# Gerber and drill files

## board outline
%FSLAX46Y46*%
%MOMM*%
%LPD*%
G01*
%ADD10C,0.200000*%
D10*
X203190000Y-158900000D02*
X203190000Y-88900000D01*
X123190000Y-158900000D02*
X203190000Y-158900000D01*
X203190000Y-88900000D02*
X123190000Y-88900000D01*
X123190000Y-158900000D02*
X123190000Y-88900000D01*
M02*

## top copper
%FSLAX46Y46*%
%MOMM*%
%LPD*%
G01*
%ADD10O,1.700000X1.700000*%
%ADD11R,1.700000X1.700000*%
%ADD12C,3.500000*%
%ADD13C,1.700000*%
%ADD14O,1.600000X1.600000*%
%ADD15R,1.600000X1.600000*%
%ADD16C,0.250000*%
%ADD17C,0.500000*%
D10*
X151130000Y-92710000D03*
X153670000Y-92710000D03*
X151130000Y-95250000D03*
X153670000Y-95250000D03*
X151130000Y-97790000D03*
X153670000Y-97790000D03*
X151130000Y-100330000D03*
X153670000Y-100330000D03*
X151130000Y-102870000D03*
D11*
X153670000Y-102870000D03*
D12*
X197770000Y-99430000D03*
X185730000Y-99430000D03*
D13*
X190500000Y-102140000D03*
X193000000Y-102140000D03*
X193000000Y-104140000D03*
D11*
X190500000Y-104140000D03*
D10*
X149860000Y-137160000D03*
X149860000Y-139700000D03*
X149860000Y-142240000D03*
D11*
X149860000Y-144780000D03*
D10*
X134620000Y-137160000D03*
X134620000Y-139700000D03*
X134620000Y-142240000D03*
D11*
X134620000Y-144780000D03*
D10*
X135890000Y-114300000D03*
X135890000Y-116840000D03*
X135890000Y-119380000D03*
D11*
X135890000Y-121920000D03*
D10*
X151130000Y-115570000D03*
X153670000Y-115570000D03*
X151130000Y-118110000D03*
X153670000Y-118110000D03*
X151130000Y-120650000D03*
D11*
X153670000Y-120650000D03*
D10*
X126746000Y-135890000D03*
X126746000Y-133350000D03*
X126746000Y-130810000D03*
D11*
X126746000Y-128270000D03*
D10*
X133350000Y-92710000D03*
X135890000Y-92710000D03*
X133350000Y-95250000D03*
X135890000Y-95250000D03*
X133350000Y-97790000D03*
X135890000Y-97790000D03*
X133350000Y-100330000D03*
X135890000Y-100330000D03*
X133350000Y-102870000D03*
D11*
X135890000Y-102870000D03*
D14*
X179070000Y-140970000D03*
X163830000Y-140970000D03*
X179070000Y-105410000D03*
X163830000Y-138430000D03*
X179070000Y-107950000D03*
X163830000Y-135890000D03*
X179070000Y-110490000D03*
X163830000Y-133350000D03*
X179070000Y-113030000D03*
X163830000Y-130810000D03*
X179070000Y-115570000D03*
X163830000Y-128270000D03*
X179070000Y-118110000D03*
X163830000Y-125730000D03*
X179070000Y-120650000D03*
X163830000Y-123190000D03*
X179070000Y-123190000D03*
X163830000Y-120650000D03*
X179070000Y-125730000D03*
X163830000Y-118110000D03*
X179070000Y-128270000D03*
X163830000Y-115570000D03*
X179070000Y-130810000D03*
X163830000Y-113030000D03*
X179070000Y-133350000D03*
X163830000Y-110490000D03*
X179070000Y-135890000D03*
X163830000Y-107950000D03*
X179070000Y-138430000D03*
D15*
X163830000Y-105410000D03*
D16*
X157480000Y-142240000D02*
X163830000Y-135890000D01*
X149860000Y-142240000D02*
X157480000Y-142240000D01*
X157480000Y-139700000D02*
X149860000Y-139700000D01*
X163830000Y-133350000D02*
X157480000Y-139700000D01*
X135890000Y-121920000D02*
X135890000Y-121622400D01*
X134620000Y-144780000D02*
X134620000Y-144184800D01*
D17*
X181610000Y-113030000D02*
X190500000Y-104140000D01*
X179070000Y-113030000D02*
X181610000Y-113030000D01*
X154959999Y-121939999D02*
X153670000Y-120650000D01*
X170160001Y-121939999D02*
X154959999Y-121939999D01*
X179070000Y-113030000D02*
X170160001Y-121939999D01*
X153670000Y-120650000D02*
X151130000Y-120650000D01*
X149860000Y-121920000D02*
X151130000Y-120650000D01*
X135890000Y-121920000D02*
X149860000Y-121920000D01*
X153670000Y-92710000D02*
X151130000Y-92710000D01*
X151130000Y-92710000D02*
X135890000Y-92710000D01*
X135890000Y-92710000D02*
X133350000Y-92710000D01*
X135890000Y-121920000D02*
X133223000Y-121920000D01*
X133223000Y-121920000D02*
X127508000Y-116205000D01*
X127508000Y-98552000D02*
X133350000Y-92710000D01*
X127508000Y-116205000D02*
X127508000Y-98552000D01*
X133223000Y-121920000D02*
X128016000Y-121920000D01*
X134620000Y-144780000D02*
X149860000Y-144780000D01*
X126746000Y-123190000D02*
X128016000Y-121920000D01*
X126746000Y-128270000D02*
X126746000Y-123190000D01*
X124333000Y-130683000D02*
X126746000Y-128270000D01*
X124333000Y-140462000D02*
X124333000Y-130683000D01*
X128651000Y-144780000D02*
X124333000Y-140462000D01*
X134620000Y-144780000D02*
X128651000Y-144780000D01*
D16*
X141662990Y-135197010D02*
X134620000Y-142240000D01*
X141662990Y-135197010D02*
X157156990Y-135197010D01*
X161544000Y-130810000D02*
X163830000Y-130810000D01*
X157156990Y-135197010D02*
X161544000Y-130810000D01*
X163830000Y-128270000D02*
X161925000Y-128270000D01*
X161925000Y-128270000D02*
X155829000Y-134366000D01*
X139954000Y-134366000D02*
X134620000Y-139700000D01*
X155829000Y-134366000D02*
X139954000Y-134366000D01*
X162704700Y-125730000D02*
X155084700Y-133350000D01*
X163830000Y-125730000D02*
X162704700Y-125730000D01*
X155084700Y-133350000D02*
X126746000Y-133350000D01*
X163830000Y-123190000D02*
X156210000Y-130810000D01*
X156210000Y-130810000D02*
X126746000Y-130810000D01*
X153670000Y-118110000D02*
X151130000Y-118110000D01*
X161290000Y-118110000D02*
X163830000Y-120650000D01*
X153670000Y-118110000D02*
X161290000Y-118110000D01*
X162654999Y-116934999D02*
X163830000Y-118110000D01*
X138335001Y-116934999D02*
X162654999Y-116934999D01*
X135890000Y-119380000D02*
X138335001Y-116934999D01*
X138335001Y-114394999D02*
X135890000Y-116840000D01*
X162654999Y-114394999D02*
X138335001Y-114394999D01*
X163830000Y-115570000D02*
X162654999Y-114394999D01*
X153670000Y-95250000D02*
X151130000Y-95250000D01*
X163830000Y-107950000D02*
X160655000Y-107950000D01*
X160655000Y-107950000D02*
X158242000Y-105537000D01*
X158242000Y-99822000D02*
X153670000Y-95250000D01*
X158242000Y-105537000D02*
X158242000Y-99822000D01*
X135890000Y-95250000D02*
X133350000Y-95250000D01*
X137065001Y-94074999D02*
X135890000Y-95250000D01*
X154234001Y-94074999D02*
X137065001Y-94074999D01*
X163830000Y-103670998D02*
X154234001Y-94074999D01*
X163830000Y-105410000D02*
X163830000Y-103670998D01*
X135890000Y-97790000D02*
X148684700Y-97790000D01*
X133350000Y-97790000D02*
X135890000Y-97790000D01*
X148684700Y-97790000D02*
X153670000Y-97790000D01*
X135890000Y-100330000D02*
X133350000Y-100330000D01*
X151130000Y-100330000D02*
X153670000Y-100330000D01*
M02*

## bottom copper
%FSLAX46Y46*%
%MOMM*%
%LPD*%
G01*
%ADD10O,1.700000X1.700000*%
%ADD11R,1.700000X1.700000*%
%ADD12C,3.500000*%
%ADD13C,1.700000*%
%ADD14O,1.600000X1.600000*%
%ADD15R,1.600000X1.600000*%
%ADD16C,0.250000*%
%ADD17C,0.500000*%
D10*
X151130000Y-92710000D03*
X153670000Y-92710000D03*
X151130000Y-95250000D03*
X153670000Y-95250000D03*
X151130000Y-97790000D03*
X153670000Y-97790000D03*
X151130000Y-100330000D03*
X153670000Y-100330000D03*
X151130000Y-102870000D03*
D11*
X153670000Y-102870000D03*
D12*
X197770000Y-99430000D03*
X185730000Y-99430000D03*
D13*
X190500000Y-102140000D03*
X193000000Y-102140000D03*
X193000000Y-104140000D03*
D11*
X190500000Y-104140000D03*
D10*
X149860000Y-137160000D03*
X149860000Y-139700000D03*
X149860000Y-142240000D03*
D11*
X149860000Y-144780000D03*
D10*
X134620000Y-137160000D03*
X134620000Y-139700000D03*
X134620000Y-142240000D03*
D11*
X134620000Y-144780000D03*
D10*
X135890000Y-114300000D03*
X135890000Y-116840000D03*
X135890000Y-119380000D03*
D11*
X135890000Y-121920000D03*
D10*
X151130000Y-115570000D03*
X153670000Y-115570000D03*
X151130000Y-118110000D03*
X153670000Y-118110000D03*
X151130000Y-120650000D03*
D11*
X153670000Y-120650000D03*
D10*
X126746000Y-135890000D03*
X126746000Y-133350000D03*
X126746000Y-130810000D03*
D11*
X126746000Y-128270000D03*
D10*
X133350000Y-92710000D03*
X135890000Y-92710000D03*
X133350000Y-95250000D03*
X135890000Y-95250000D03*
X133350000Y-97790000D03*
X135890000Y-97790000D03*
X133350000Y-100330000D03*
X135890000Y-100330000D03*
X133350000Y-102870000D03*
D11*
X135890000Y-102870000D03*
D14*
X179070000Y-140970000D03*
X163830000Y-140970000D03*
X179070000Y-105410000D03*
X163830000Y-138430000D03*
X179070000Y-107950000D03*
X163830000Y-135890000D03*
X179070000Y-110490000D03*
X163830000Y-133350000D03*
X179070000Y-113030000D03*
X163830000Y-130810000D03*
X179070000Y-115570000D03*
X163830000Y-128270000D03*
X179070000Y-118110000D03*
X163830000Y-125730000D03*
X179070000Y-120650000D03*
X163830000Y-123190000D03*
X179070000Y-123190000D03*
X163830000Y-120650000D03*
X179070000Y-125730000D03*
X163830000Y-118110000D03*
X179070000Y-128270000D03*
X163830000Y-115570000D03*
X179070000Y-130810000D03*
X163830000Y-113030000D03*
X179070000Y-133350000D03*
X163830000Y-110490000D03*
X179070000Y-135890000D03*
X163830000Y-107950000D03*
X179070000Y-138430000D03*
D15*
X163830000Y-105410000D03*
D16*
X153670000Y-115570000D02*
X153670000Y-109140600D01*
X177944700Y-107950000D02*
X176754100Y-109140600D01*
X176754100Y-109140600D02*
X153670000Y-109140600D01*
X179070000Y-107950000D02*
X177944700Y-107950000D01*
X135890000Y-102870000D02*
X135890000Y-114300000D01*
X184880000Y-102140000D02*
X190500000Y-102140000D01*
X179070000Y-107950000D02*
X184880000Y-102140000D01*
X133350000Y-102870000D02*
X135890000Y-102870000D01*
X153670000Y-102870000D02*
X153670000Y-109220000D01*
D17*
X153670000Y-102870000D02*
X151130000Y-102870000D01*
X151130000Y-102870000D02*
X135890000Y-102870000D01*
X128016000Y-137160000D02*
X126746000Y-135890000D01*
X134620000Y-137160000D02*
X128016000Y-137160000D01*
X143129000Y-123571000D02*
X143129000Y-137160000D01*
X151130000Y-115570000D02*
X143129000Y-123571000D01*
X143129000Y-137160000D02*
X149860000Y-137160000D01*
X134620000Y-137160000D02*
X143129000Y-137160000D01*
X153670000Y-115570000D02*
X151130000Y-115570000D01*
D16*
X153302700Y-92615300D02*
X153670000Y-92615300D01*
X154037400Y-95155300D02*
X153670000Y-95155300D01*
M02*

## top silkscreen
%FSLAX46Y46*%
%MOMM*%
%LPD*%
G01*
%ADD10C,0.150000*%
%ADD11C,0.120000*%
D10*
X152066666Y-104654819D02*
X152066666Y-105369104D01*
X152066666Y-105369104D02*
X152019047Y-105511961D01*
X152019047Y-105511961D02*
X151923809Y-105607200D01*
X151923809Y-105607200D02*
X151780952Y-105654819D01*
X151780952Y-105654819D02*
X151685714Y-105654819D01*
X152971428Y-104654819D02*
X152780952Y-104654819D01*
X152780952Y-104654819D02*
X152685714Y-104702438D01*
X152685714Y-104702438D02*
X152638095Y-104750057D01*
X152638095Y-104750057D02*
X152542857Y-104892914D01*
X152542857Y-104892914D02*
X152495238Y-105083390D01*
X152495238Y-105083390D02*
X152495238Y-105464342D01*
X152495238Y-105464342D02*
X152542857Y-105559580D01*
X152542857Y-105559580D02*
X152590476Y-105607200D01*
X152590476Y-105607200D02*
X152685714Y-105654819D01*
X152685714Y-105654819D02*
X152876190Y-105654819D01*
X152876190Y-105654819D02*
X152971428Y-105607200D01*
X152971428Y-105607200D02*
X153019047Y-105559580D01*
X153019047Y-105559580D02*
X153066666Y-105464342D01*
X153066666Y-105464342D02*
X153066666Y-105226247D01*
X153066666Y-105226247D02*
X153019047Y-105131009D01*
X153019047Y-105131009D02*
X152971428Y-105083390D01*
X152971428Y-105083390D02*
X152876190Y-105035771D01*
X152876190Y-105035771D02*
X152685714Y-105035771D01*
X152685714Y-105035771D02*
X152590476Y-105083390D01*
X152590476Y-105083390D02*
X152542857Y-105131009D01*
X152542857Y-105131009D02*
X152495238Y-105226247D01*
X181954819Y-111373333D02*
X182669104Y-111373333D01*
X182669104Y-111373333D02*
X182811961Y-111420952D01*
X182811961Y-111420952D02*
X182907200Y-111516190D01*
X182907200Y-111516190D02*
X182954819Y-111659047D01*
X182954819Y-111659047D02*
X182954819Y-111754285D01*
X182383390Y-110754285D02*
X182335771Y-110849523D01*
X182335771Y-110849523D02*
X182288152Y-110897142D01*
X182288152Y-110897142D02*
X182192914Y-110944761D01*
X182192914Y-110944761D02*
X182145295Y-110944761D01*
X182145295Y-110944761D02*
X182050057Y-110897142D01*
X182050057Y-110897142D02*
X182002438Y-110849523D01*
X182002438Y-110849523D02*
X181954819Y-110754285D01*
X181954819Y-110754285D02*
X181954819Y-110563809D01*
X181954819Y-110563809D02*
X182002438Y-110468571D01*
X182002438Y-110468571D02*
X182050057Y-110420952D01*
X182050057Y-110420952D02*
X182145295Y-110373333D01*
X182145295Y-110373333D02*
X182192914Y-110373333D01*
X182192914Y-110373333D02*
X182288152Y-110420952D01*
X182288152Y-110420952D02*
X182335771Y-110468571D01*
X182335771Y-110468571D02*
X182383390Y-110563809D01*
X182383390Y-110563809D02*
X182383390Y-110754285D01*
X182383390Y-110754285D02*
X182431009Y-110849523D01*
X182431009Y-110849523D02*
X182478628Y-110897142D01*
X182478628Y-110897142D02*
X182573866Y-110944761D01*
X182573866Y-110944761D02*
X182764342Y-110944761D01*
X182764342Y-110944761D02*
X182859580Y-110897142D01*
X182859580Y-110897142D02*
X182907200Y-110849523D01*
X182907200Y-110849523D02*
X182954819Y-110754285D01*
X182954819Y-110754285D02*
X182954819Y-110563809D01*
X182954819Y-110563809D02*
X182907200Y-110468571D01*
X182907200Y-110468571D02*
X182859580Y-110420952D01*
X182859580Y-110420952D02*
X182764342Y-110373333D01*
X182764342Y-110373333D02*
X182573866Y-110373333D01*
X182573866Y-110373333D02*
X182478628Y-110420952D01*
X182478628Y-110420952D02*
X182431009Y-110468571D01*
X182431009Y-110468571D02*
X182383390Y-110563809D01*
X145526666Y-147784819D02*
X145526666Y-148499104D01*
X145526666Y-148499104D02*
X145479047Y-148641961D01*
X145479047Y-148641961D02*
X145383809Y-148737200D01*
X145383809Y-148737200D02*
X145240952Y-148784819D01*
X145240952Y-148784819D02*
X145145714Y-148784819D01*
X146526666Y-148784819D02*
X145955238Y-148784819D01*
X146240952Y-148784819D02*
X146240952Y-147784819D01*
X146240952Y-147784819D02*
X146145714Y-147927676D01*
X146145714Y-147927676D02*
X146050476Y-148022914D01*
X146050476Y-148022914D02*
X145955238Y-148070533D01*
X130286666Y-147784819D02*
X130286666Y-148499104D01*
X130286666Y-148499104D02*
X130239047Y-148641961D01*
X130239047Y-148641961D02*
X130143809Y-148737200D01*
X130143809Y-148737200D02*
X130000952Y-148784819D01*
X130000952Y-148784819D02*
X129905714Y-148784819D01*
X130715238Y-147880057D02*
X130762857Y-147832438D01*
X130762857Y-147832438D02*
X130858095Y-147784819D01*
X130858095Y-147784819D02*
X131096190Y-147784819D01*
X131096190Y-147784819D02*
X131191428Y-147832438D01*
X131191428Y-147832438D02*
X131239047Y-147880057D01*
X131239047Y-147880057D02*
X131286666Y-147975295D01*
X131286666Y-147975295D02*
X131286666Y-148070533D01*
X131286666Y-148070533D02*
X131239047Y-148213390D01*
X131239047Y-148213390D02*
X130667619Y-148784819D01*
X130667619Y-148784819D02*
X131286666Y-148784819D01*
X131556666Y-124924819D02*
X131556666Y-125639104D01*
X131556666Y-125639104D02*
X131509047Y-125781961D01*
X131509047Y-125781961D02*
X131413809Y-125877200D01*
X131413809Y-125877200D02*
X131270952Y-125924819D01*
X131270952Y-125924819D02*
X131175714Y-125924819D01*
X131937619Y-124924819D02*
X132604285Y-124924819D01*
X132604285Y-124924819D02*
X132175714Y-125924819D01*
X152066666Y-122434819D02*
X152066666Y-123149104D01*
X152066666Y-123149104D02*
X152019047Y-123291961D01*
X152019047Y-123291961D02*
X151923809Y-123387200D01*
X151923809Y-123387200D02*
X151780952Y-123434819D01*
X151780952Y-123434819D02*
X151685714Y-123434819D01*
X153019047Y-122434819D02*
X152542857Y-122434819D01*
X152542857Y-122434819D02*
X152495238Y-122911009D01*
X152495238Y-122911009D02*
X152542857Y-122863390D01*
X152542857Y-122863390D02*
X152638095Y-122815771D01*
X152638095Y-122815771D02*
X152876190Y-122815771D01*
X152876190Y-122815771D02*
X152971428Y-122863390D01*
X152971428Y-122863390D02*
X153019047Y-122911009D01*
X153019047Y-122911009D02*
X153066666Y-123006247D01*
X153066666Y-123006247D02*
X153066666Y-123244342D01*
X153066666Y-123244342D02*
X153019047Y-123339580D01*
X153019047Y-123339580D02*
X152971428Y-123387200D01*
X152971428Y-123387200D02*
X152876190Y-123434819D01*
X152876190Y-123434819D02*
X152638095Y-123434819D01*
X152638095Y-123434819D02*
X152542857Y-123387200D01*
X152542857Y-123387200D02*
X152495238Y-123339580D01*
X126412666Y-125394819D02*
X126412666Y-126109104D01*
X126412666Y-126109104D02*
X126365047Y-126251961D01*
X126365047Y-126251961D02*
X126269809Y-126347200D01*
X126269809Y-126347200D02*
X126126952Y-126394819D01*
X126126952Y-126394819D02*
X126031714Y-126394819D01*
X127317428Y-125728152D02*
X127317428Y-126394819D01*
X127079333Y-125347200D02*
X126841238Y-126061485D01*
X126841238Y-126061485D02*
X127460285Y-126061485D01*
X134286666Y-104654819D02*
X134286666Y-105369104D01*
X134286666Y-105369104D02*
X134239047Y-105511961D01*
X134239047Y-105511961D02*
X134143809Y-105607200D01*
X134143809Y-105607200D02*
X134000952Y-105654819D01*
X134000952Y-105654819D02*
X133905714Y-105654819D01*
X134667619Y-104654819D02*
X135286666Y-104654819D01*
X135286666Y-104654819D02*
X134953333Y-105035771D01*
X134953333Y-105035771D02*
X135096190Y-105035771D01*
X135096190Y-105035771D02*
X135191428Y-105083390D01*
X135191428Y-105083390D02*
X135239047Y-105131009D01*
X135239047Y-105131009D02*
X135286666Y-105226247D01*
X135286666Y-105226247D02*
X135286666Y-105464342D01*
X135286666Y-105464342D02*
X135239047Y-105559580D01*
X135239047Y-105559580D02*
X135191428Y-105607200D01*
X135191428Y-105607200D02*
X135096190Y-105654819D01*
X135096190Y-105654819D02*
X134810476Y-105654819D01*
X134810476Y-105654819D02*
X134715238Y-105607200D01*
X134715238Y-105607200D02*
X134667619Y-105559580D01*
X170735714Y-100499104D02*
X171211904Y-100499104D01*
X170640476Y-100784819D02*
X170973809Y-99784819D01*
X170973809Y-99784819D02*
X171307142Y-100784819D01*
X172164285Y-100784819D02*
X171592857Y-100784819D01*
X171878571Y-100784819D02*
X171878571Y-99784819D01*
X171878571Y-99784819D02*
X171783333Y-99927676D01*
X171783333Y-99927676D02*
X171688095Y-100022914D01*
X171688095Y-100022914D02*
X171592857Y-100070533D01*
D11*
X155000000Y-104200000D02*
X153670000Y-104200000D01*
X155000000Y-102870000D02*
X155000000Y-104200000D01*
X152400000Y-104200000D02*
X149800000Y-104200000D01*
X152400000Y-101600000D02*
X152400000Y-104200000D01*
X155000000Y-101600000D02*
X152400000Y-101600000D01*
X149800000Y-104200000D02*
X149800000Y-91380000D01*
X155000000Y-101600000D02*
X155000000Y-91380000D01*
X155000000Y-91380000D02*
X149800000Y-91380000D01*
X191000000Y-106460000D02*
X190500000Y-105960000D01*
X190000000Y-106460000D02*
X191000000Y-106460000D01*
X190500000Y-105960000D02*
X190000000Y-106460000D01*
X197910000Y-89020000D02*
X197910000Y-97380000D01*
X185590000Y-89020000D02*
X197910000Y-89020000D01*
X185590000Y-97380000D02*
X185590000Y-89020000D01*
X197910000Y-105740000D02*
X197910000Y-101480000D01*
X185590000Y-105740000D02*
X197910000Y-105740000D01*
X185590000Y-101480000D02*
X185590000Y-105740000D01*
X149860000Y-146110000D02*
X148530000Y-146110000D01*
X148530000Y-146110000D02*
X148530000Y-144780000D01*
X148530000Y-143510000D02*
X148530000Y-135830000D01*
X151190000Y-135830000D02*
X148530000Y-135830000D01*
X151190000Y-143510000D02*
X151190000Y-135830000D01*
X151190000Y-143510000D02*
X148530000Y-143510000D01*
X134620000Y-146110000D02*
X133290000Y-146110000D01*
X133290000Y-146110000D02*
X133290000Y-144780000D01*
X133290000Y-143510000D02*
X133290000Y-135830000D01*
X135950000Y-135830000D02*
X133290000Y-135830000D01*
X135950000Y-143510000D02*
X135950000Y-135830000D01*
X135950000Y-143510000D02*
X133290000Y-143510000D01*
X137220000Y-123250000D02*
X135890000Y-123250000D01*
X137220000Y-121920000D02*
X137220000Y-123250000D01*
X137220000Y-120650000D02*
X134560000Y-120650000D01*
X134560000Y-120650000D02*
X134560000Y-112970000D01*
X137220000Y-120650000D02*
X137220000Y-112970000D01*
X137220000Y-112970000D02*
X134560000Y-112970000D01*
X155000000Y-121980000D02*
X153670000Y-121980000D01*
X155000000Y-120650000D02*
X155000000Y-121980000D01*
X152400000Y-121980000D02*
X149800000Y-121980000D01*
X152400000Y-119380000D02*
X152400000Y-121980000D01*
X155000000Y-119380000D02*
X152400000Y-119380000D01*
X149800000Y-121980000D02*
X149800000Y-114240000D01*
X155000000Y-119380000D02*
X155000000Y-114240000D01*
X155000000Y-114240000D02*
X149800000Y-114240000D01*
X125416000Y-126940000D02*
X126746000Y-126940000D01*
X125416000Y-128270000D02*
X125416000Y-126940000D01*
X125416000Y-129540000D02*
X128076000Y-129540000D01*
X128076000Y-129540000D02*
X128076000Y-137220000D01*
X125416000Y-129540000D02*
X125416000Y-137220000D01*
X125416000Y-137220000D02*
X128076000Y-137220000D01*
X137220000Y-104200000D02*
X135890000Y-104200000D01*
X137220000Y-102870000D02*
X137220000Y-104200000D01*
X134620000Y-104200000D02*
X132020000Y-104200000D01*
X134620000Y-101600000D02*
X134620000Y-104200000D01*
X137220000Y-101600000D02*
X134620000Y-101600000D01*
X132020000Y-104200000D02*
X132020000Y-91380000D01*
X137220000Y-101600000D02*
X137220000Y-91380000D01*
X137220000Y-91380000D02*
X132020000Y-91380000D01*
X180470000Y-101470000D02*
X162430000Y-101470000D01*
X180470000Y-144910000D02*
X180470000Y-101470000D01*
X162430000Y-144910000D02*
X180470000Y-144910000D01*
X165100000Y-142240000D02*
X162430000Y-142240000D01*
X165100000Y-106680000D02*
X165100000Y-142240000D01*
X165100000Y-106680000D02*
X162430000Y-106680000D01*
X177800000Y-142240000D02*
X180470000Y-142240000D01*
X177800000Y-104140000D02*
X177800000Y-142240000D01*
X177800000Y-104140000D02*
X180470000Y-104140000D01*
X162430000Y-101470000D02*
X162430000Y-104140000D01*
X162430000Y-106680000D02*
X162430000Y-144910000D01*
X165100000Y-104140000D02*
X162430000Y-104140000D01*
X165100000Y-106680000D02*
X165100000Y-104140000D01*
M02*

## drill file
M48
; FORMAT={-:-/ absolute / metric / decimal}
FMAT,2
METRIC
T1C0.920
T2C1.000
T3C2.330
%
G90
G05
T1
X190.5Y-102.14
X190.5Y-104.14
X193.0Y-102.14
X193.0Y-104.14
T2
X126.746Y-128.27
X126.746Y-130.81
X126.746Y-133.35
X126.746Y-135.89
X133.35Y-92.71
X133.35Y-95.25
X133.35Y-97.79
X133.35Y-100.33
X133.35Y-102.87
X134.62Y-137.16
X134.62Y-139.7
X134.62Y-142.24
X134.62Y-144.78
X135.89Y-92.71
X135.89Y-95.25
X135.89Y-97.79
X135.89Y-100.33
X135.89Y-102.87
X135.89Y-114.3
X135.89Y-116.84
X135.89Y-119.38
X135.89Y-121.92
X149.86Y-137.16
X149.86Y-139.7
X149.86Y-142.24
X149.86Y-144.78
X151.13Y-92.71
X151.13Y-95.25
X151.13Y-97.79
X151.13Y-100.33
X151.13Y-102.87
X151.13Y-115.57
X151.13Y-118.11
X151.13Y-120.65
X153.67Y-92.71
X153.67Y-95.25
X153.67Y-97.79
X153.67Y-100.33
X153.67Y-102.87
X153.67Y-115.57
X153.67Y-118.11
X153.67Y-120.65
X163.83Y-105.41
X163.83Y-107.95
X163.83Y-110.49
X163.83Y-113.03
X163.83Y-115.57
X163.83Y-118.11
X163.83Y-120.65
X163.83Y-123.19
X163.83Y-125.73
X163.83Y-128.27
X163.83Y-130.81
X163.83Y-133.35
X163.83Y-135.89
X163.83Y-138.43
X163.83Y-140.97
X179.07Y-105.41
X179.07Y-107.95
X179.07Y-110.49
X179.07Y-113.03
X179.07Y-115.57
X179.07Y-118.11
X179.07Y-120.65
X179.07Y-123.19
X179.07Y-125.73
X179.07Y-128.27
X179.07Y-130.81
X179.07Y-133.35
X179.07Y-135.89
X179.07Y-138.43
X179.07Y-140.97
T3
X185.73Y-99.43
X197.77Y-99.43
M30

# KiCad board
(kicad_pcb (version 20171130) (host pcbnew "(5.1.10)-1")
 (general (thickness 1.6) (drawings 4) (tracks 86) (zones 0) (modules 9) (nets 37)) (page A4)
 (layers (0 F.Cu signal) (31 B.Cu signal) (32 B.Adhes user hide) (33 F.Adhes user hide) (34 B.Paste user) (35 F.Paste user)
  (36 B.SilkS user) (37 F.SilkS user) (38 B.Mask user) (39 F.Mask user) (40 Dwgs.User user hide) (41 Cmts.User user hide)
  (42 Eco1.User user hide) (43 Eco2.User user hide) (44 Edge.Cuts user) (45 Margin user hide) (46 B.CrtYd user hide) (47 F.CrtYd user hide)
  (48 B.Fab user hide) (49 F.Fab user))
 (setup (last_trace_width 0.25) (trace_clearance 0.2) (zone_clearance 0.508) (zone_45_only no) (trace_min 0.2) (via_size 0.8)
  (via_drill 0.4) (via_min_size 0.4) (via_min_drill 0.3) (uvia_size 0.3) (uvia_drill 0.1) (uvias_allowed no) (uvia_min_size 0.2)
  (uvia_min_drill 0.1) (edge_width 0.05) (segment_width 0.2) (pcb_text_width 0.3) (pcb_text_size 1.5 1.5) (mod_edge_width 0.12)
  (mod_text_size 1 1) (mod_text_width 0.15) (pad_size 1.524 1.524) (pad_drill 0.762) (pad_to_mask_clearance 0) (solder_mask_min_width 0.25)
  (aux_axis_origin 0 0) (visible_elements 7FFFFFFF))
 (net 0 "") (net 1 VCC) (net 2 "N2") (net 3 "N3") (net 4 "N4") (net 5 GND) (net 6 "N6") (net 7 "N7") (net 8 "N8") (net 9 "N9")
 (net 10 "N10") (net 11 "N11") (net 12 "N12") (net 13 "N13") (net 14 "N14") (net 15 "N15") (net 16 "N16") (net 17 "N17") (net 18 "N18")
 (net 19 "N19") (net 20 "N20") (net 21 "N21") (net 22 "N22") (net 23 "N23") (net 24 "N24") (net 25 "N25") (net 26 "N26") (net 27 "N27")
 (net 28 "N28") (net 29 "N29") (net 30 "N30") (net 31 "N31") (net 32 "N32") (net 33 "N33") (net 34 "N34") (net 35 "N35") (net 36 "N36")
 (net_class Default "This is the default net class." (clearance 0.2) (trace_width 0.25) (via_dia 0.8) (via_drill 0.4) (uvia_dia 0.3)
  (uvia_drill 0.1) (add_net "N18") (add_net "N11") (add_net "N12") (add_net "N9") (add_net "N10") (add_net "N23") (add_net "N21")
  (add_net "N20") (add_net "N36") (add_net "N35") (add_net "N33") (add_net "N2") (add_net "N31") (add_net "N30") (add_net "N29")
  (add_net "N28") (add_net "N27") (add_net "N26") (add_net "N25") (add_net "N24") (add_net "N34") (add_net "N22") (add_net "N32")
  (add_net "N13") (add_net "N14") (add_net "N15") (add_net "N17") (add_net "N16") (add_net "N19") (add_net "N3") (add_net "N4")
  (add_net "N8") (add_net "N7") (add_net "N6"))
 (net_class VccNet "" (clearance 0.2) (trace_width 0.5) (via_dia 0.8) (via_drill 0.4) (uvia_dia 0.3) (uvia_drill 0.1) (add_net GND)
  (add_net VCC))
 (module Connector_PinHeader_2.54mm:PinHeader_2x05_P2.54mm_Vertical (layer F.Cu) (at 153.67 102.87 180)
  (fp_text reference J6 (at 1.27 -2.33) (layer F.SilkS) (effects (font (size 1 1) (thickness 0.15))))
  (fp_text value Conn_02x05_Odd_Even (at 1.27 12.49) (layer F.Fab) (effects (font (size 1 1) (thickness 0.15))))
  (fp_line (start -1.33 -1.33) (end 0 -1.33) (layer F.SilkS) (width 0.12))
  (fp_line (start -1.33 0) (end -1.33 -1.33) (layer F.SilkS) (width 0.12))
  (fp_line (start 1.27 -1.33) (end 3.87 -1.33) (layer F.SilkS) (width 0.12))
  (fp_line (start 1.27 1.27) (end 1.27 -1.33) (layer F.SilkS) (width 0.12))
  (fp_line (start -1.33 1.27) (end 1.27 1.27) (layer F.SilkS) (width 0.12))
  (fp_line (start 3.87 -1.33) (end 3.87 11.49) (layer F.SilkS) (width 0.12))
  (fp_line (start -1.33 1.27) (end -1.33 11.49) (layer F.SilkS) (width 0.12))
  (fp_line (start -1.33 11.49) (end 3.87 11.49) (layer F.SilkS) (width 0.12))
  (pad 10 thru_hole oval (at 2.54 10.16 180) (size 1.7 1.7) (drill 1) (layers *.Cu *.Mask) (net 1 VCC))
  (pad 9 thru_hole oval (at 0 10.16 180) (size 1.7 1.7) (drill 1) (layers *.Cu *.Mask) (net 1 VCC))
  (pad 8 thru_hole oval (at 2.54 7.62 180) (size 1.7 1.7) (drill 1) (layers *.Cu *.Mask) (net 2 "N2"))
  (pad 7 thru_hole oval (at 0 7.62 180) (size 1.7 1.7) (drill 1) (layers *.Cu *.Mask) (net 2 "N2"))
  (pad 6 thru_hole oval (at 2.54 5.08 180) (size 1.7 1.7) (drill 1) (layers *.Cu *.Mask) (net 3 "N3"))
  (pad 5 thru_hole oval (at 0 5.08 180) (size 1.7 1.7) (drill 1) (layers *.Cu *.Mask) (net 3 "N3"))
  (pad 4 thru_hole oval (at 2.54 2.54 180) (size 1.7 1.7) (drill 1) (layers *.Cu *.Mask) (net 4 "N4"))
  (pad 3 thru_hole oval (at 0 2.54 180) (size 1.7 1.7) (drill 1) (layers *.Cu *.Mask) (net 4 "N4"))
  (pad 2 thru_hole oval (at 2.54 0 180) (size 1.7 1.7) (drill 1) (layers *.Cu *.Mask) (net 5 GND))
  (pad 1 thru_hole rect (at 0 0 180) (size 1.7 1.7) (drill 1) (layers *.Cu *.Mask) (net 5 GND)))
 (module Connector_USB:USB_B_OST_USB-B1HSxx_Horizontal (layer F.Cu) (at 190.5 104.14 90)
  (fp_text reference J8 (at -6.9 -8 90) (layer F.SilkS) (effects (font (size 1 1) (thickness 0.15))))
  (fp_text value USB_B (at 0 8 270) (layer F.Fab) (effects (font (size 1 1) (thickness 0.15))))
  (fp_line (start -2.32 0.5) (end -1.82 0) (layer F.SilkS) (width 0.12))
  (fp_line (start -2.32 -0.5) (end -2.32 0.5) (layer F.SilkS) (width 0.12))
  (fp_line (start -1.82 0) (end -2.32 -0.5) (layer F.SilkS) (width 0.12))
  (fp_line (start 15.12 7.41) (end 6.76 7.41) (layer F.SilkS) (width 0.12))
  (fp_line (start 15.12 -4.91) (end 15.12 7.41) (layer F.SilkS) (width 0.12))
  (fp_line (start 6.76 -4.91) (end 15.12 -4.91) (layer F.SilkS) (width 0.12))
  (fp_line (start -1.6 7.41) (end 2.66 7.41) (layer F.SilkS) (width 0.12))
  (fp_line (start -1.6 -4.91) (end -1.6 7.41) (layer F.SilkS) (width 0.12))
  (fp_line (start 2.66 -4.91) (end -1.6 -4.91) (layer F.SilkS) (width 0.12))
  (pad 5 thru_hole circle (at 4.71 7.27 90) (size 3.5 3.5) (drill 2.33) (layers *.Cu *.Mask) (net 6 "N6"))
  (pad 5 thru_hole circle (at 4.71 -4.77 90) (size 3.5 3.5) (drill 2.33) (layers *.Cu *.Mask) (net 6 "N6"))
  (pad 4 thru_hole circle (at 2 0 90) (size 1.7 1.7) (drill 0.92) (layers *.Cu *.Mask) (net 5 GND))
  (pad 3 thru_hole circle (at 2 2.5 90) (size 1.7 1.7) (drill 0.92) (layers *.Cu *.Mask) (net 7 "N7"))
  (pad 2 thru_hole circle (at 0 2.5 90) (size 1.7 1.7) (drill 0.92) (layers *.Cu *.Mask) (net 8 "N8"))
  (pad 1 thru_hole rect (at 0 0 90) (size 1.7 1.7) (drill 0.92) (layers *.Cu *.Mask) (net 1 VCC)))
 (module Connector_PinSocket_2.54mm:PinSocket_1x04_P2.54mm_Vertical (layer F.Cu) (at 149.86 144.78 180)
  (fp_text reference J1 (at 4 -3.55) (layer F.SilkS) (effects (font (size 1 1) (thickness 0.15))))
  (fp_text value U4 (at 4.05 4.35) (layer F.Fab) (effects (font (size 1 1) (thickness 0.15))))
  (fp_line (start 0 -1.33) (end 1.33 -1.33) (layer F.SilkS) (width 0.12))
  (fp_line (start 1.33 -1.33) (end 1.33 0) (layer F.SilkS) (width 0.12))
  (fp_line (start 1.33 1.27) (end 1.33 8.95) (layer F.SilkS) (width 0.12))
  (fp_line (start -1.33 8.95) (end 1.33 8.95) (layer F.SilkS) (width 0.12))
  (fp_line (start -1.33 1.27) (end -1.33 8.95) (layer F.SilkS) (width 0.12))
  (fp_line (start -1.33 1.27) (end 1.33 1.27) (layer F.SilkS) (width 0.12))
  (pad 4 thru_hole oval (at 0 7.62 180) (size 1.7 1.7) (drill 1) (layers *.Cu *.Mask) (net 5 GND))
  (pad 3 thru_hole oval (at 0 5.08 180) (size 1.7 1.7) (drill 1) (layers *.Cu *.Mask) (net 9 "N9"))
  (pad 2 thru_hole oval (at 0 2.54 180) (size 1.7 1.7) (drill 1) (layers *.Cu *.Mask) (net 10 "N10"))
  (pad 1 thru_hole rect (at 0 0 180) (size 1.7 1.7) (drill 1) (layers *.Cu *.Mask) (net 1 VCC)))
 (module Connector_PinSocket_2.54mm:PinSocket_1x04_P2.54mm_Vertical (layer F.Cu) (at 134.62 144.78 180)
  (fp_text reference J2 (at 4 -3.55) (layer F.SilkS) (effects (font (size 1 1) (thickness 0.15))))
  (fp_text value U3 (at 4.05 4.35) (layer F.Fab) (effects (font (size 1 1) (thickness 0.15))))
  (fp_line (start 0 -1.33) (end 1.33 -1.33) (layer F.SilkS) (width 0.12))
  (fp_line (start 1.33 -1.33) (end 1.33 0) (layer F.SilkS) (width 0.12))
  (fp_line (start 1.33 1.27) (end 1.33 8.95) (layer F.SilkS) (width 0.12))
  (fp_line (start -1.33 8.95) (end 1.33 8.95) (layer F.SilkS) (width 0.12))
  (fp_line (start -1.33 1.27) (end -1.33 8.95) (layer F.SilkS) (width 0.12))
  (fp_line (start -1.33 1.27) (end 1.33 1.27) (layer F.SilkS) (width 0.12))
  (pad 4 thru_hole oval (at 0 7.62 180) (size 1.7 1.7) (drill 1) (layers *.Cu *.Mask) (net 5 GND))
  (pad 3 thru_hole oval (at 0 5.08 180) (size 1.7 1.7) (drill 1) (layers *.Cu *.Mask) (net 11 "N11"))
  (pad 2 thru_hole oval (at 0 2.54 180) (size 1.7 1.7) (drill 1) (layers *.Cu *.Mask) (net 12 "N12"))
  (pad 1 thru_hole rect (at 0 0 180) (size 1.7 1.7) (drill 1) (layers *.Cu *.Mask) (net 1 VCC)))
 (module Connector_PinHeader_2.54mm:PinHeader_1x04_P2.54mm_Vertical (layer F.Cu) (at 135.89 121.92 180)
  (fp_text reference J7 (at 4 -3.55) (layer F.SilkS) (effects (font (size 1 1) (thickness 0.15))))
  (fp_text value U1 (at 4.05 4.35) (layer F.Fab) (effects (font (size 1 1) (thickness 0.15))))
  (fp_line (start -1.33 -1.33) (end 0 -1.33) (layer F.SilkS) (width 0.12))
  (fp_line (start -1.33 0) (end -1.33 -1.33) (layer F.SilkS) (width 0.12))
  (fp_line (start -1.33 1.27) (end 1.33 1.27) (layer F.SilkS) (width 0.12))
  (fp_line (start 1.33 1.27) (end 1.33 8.95) (layer F.SilkS) (width 0.12))
  (fp_line (start -1.33 1.27) (end -1.33 8.95) (layer F.SilkS) (width 0.12))
  (fp_line (start -1.33 8.95) (end 1.33 8.95) (layer F.SilkS) (width 0.12))
  (pad 4 thru_hole oval (at 0 7.62 180) (size 1.7 1.7) (drill 1) (layers *.Cu *.Mask) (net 5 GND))
  (pad 3 thru_hole oval (at 0 5.08 180) (size 1.7 1.7) (drill 1) (layers *.Cu *.Mask) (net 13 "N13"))
  (pad 2 thru_hole oval (at 0 2.54 180) (size 1.7 1.7) (drill 1) (layers *.Cu *.Mask) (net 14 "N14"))
  (pad 1 thru_hole rect (at 0 0 180) (size 1.7 1.7) (drill 1) (layers *.Cu *.Mask) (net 1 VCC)))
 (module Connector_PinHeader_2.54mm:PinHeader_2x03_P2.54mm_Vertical (layer F.Cu) (at 153.67 120.65 180)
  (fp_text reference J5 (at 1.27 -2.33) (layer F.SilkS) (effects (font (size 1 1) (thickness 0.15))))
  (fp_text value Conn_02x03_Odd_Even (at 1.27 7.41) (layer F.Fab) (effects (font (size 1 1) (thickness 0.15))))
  (fp_line (start -1.33 -1.33) (end 0 -1.33) (layer F.SilkS) (width 0.12))
  (fp_line (start -1.33 0) (end -1.33 -1.33) (layer F.SilkS) (width 0.12))
  (fp_line (start 1.27 -1.33) (end 3.87 -1.33) (layer F.SilkS) (width 0.12))
  (fp_line (start 1.27 1.27) (end 1.27 -1.33) (layer F.SilkS) (width 0.12))
  (fp_line (start -1.33 1.27) (end 1.27 1.27) (layer F.SilkS) (width 0.12))
  (fp_line (start 3.87 -1.33) (end 3.87 6.41) (layer F.SilkS) (width 0.12))
  (fp_line (start -1.33 1.27) (end -1.33 6.41) (layer F.SilkS) (width 0.12))
  (fp_line (start -1.33 6.41) (end 3.87 6.41) (layer F.SilkS) (width 0.12))
  (pad 6 thru_hole oval (at 2.54 5.08 180) (size 1.7 1.7) (drill 1) (layers *.Cu *.Mask) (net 5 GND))
  (pad 5 thru_hole oval (at 0 5.08 180) (size 1.7 1.7) (drill 1) (layers *.Cu *.Mask) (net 5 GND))
  (pad 4 thru_hole oval (at 2.54 2.54 180) (size 1.7 1.7) (drill 1) (layers *.Cu *.Mask) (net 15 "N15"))
  (pad 3 thru_hole oval (at 0 2.54 180) (size 1.7 1.7) (drill 1) (layers *.Cu *.Mask) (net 15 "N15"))
  (pad 2 thru_hole oval (at 2.54 0 180) (size 1.7 1.7) (drill 1) (layers *.Cu *.Mask) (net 1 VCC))
  (pad 1 thru_hole rect (at 0 0 180) (size 1.7 1.7) (drill 1) (layers *.Cu *.Mask) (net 1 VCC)))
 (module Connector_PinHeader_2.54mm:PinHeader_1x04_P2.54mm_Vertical (layer F.Cu) (at 126.746 128.27)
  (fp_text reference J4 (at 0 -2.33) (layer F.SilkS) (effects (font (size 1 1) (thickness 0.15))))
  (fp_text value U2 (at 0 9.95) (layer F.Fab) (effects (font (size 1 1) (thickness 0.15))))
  (fp_line (start -1.33 -1.33) (end 0 -1.33) (layer F.SilkS) (width 0.12))
  (fp_line (start -1.33 0) (end -1.33 -1.33) (layer F.SilkS) (width 0.12))
  (fp_line (start -1.33 1.27) (end 1.33 1.27) (layer F.SilkS) (width 0.12))
  (fp_line (start 1.33 1.27) (end 1.33 8.95) (layer F.SilkS) (width 0.12))
  (fp_line (start -1.33 1.27) (end -1.33 8.95) (layer F.SilkS) (width 0.12))
  (fp_line (start -1.33 8.95) (end 1.33 8.95) (layer F.SilkS) (width 0.12))
  (pad 4 thru_hole oval (at 0 7.62) (size 1.7 1.7) (drill 1) (layers *.Cu *.Mask) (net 5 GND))
  (pad 3 thru_hole oval (at 0 5.08) (size 1.7 1.7) (drill 1) (layers *.Cu *.Mask) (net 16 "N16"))
  (pad 2 thru_hole oval (at 0 2.54) (size 1.7 1.7) (drill 1) (layers *.Cu *.Mask) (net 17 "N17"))
  (pad 1 thru_hole rect (at 0 0) (size 1.7 1.7) (drill 1) (layers *.Cu *.Mask) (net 1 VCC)))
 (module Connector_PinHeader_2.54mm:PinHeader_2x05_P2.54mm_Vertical (layer F.Cu) (at 135.89 102.87 180)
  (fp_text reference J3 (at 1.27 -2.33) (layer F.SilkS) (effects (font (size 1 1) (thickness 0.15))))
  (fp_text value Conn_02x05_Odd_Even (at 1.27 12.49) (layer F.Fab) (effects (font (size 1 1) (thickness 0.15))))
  (fp_line (start -1.33 -1.33) (end 0 -1.33) (layer F.SilkS) (width 0.12))
  (fp_line (start -1.33 0) (end -1.33 -1.33) (layer F.SilkS) (width 0.12))
  (fp_line (start 1.27 -1.33) (end 3.87 -1.33) (layer F.SilkS) (width 0.12))
  (fp_line (start 1.27 1.27) (end 1.27 -1.33) (layer F.SilkS) (width 0.12))
  (fp_line (start -1.33 1.27) (end 1.27 1.27) (layer F.SilkS) (width 0.12))
  (fp_line (start 3.87 -1.33) (end 3.87 11.49) (layer F.SilkS) (width 0.12))
  (fp_line (start -1.33 1.27) (end -1.33 11.49) (layer F.SilkS) (width 0.12))
  (fp_line (start -1.33 11.49) (end 3.87 11.49) (layer F.SilkS) (width 0.12))
  (pad 10 thru_hole oval (at 2.54 10.16 180) (size 1.7 1.7) (drill 1) (layers *.Cu *.Mask) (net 1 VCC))
  (pad 9 thru_hole oval (at 0 10.16 180) (size 1.7 1.7) (drill 1) (layers *.Cu *.Mask) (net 1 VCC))
  (pad 8 thru_hole oval (at 2.54 7.62 180) (size 1.7 1.7) (drill 1) (layers *.Cu *.Mask) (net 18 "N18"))
  (pad 7 thru_hole oval (at 0 7.62 180) (size 1.7 1.7) (drill 1) (layers *.Cu *.Mask) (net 18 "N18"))
  (pad 6 thru_hole oval (at 2.54 5.08 180) (size 1.7 1.7) (drill 1) (layers *.Cu *.Mask) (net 3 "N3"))
  (pad 5 thru_hole oval (at 0 5.08 180) (size 1.7 1.7) (drill 1) (layers *.Cu *.Mask) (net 3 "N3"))
  (pad 4 thru_hole oval (at 2.54 2.54 180) (size 1.7 1.7) (drill 1) (layers *.Cu *.Mask) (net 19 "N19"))
  (pad 3 thru_hole oval (at 0 2.54 180) (size 1.7 1.7) (drill 1) (layers *.Cu *.Mask) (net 19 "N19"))
  (pad 2 thru_hole oval (at 2.54 0 180) (size 1.7 1.7) (drill 1) (layers *.Cu *.Mask) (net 5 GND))
  (pad 1 thru_hole rect (at 0 0 180) (size 1.7 1.7) (drill 1) (layers *.Cu *.Mask) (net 5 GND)))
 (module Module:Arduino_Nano (layer F.Cu) (at 163.83 105.41)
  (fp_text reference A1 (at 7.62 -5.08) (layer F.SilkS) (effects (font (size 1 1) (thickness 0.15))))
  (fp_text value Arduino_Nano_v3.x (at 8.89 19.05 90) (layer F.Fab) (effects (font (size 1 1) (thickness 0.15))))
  (fp_line (start 16.64 -3.94) (end -1.4 -3.94) (layer F.SilkS) (width 0.12))
  (fp_line (start 16.64 39.5) (end 16.64 -3.94) (layer F.SilkS) (width 0.12))
  (fp_line (start -1.4 39.5) (end 16.64 39.5) (layer F.SilkS) (width 0.12))
  (fp_line (start 1.27 36.83) (end -1.4 36.83) (layer F.SilkS) (width 0.12))
  (fp_line (start 1.27 1.27) (end 1.27 36.83) (layer F.SilkS) (width 0.12))
  (fp_line (start 1.27 1.27) (end -1.4 1.27) (layer F.SilkS) (width 0.12))
  (fp_line (start 13.97 36.83) (end 16.64 36.83) (layer F.SilkS) (width 0.12))
  (fp_line (start 13.97 -1.27) (end 13.97 36.83) (layer F.SilkS) (width 0.12))
  (fp_line (start 13.97 -1.27) (end 16.64 -1.27) (layer F.SilkS) (width 0.12))
  (fp_line (start -1.4 -3.94) (end -1.4 -1.27) (layer F.SilkS) (width 0.12))
  (fp_line (start -1.4 1.27) (end -1.4 39.5) (layer F.SilkS) (width 0.12))
  (fp_line (start 1.27 -1.27) (end -1.4 -1.27) (layer F.SilkS) (width 0.12))
  (fp_line (start 1.27 1.27) (end 1.27 -1.27) (layer F.SilkS) (width 0.12))
  (pad 16 thru_hole oval (at 15.24 35.56) (size 1.6 1.6) (drill 1) (layers *.Cu *.Mask) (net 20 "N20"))
  (pad 15 thru_hole oval (at 0 35.56) (size 1.6 1.6) (drill 1) (layers *.Cu *.Mask) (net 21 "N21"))
  (pad 30 thru_hole oval (at 15.24 0) (size 1.6 1.6) (drill 1) (layers *.Cu *.Mask) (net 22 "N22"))
  (pad 14 thru_hole oval (at 0 33.02) (size 1.6 1.6) (drill 1) (layers *.Cu *.Mask) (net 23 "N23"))
  (pad 29 thru_hole oval (at 15.24 2.54) (size 1.6 1.6) (drill 1) (layers *.Cu *.Mask) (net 5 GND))
  (pad 13 thru_hole oval (at 0 30.48) (size 1.6 1.6) (drill 1) (layers *.Cu *.Mask) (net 10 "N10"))
  (pad 28 thru_hole oval (at 15.24 5.08) (size 1.6 1.6) (drill 1) (layers *.Cu *.Mask) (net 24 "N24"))
  (pad 12 thru_hole oval (at 0 27.94) (size 1.6 1.6) (drill 1) (layers *.Cu *.Mask) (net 9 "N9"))
  (pad 27 thru_hole oval (at 15.24 7.62) (size 1.6 1.6) (drill 1) (layers *.Cu *.Mask) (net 1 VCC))
  (pad 11 thru_hole oval (at 0 25.4) (size 1.6 1.6) (drill 1) (layers *.Cu *.Mask) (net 12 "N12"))
  (pad 26 thru_hole oval (at 15.24 10.16) (size 1.6 1.6) (drill 1) (layers *.Cu *.Mask) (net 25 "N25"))
  (pad 10 thru_hole oval (at 0 22.86) (size 1.6 1.6) (drill 1) (layers *.Cu *.Mask) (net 11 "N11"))
  (pad 25 thru_hole oval (at 15.24 12.7) (size 1.6 1.6) (drill 1) (layers *.Cu *.Mask) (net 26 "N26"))
  (pad 9 thru_hole oval (at 0 20.32) (size 1.6 1.6) (drill 1) (layers *.Cu *.Mask) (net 16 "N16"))
  (pad 24 thru_hole oval (at 15.24 15.24) (size 1.6 1.6) (drill 1) (layers *.Cu *.Mask) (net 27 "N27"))
  (pad 8 thru_hole oval (at 0 17.78) (size 1.6 1.6) (drill 1) (layers *.Cu *.Mask) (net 17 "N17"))
  (pad 23 thru_hole oval (at 15.24 17.78) (size 1.6 1.6) (drill 1) (layers *.Cu *.Mask) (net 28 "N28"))
  (pad 7 thru_hole oval (at 0 15.24) (size 1.6 1.6) (drill 1) (layers *.Cu *.Mask) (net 15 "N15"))
  (pad 22 thru_hole oval (at 15.24 20.32) (size 1.6 1.6) (drill 1) (layers *.Cu *.Mask) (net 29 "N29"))
  (pad 6 thru_hole oval (at 0 12.7) (size 1.6 1.6) (drill 1) (layers *.Cu *.Mask) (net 14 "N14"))
  (pad 21 thru_hole oval (at 15.24 22.86) (size 1.6 1.6) (drill 1) (layers *.Cu *.Mask) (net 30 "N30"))
  (pad 5 thru_hole oval (at 0 10.16) (size 1.6 1.6) (drill 1) (layers *.Cu *.Mask) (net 13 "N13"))
  (pad 20 thru_hole oval (at 15.24 25.4) (size 1.6 1.6) (drill 1) (layers *.Cu *.Mask) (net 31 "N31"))
  (pad 4 thru_hole oval (at 0 7.62) (size 1.6 1.6) (drill 1) (layers *.Cu *.Mask) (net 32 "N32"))
  (pad 19 thru_hole oval (at 15.24 27.94) (size 1.6 1.6) (drill 1) (layers *.Cu *.Mask) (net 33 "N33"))
  (pad 3 thru_hole oval (at 0 5.08) (size 1.6 1.6) (drill 1) (layers *.Cu *.Mask) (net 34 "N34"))
  (pad 18 thru_hole oval (at 15.24 30.48) (size 1.6 1.6) (drill 1) (layers *.Cu *.Mask) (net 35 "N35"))
  (pad 2 thru_hole oval (at 0 2.54) (size 1.6 1.6) (drill 1) (layers *.Cu *.Mask) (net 2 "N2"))
  (pad 17 thru_hole oval (at 15.24 33.02) (size 1.6 1.6) (drill 1) (layers *.Cu *.Mask) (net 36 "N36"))
  (pad 1 thru_hole rect (at 0 0) (size 1.6 1.6) (drill 1) (layers *.Cu *.Mask) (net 18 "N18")))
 (gr_line (start 203.19 158.9) (end 203.19 88.9) (layer Edge.Cuts) (width 0.2))
 (gr_line (start 123.19 158.9) (end 203.19 158.9) (layer Edge.Cuts) (width 0.2))
 (gr_line (start 203.19 88.9) (end 123.19 88.9) (layer Edge.Cuts) (width 0.2))
 (gr_line (start 123.19 158.9) (end 123.19 88.9) (layer Edge.Cuts) (width 0.2))
 (segment (start 153.67 115.57) (end 153.67 109.1406) (width 0.25) (layer B.Cu) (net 5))
 (segment (start 177.9447 107.95) (end 176.7541 109.1406) (width 0.25) (layer B.Cu) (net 5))
 (segment (start 176.7541 109.1406) (end 153.67 109.1406) (width 0.25) (layer B.Cu) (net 5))
 (segment (start 179.07 107.95) (end 177.9447 107.95) (width 0.25) (layer B.Cu) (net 5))
 (segment (start 135.89 102.87) (end 135.89 114.3) (width 0.25) (layer B.Cu) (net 5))
 (segment (start 184.88 102.14) (end 190.5 102.14) (width 0.25) (layer B.Cu) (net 5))
 (segment (start 179.07 107.95) (end 184.88 102.14) (width 0.25) (layer B.Cu) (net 5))
 (segment (start 133.35 102.87) (end 135.89 102.87) (width 0.25) (layer B.Cu) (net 5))
 (segment (start 153.67 102.87) (end 153.67 109.22) (width 0.25) (layer B.Cu) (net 5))
 (segment (start 153.67 102.87) (end 151.13 102.87) (width 0.5) (layer B.Cu) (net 5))
 (segment (start 151.13 102.87) (end 135.89 102.87) (width 0.5) (layer B.Cu) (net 5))
 (segment (start 128.016 137.16) (end 126.746 135.89) (width 0.5) (layer B.Cu) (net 5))
 (segment (start 134.62 137.16) (end 128.016 137.16) (width 0.5) (layer B.Cu) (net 5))
 (segment (start 143.129 123.571) (end 143.129 137.16) (width 0.5) (layer B.Cu) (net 5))
 (segment (start 151.13 115.57) (end 143.129 123.571) (width 0.5) (layer B.Cu) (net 5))
 (segment (start 143.129 137.16) (end 149.86 137.16) (width 0.5) (layer B.Cu) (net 5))
 (segment (start 134.62 137.16) (end 143.129 137.16) (width 0.5) (layer B.Cu) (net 5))
 (segment (start 153.67 115.57) (end 151.13 115.57) (width 0.5) (layer B.Cu) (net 5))
 (segment (start 157.48 142.24) (end 163.83 135.89) (width 0.25) (layer F.Cu) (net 10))
 (segment (start 149.86 142.24) (end 157.48 142.24) (width 0.25) (layer F.Cu) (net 10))
 (segment (start 157.48 139.7) (end 149.86 139.7) (width 0.25) (layer F.Cu) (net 9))
 (segment (start 163.83 133.35) (end 157.48 139.7) (width 0.25) (layer F.Cu) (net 9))
 (segment (start 135.89 121.92) (end 135.89 121.6224) (width 0.25) (layer F.Cu) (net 1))
 (segment (start 153.3027 92.6153) (end 153.67 92.6153) (width 0.25) (layer B.Cu) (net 1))
 (segment (start 134.62 144.78) (end 134.62 144.1848) (width 0.25) (layer F.Cu) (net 1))
 (segment (start 181.61 113.03) (end 190.5 104.14) (width 0.5) (layer F.Cu) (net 1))
 (segment (start 179.07 113.03) (end 181.61 113.03) (width 0.5) (layer F.Cu) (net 1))
 (segment (start 154.959999 121.939999) (end 153.67 120.65) (width 0.5) (layer F.Cu) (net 1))
 (segment (start 170.160001 121.939999) (end 154.959999 121.939999) (width 0.5) (layer F.Cu) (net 1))
 (segment (start 179.07 113.03) (end 170.160001 121.939999) (width 0.5) (layer F.Cu) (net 1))
 (segment (start 153.67 120.65) (end 151.13 120.65) (width 0.5) (layer F.Cu) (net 1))
 (segment (start 149.86 121.92) (end 151.13 120.65) (width 0.5) (layer F.Cu) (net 1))
 (segment (start 135.89 121.92) (end 149.86 121.92) (width 0.5) (layer F.Cu) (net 1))
 (segment (start 153.67 92.71) (end 151.13 92.71) (width 0.5) (layer F.Cu) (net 1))
 (segment (start 151.13 92.71) (end 135.89 92.71) (width 0.5) (layer F.Cu) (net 1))
 (segment (start 135.89 92.71) (end 133.35 92.71) (width 0.5) (layer F.Cu) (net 1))
 (segment (start 135.89 121.92) (end 133.223 121.92) (width 0.5) (layer F.Cu) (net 1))
 (segment (start 133.223 121.92) (end 127.508 116.205) (width 0.5) (layer F.Cu) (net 1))
 (segment (start 127.508 98.552) (end 133.35 92.71) (width 0.5) (layer F.Cu) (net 1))
 (segment (start 127.508 116.205) (end 127.508 98.552) (width 0.5) (layer F.Cu) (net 1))
 (segment (start 133.223 121.92) (end 128.016 121.92) (width 0.5) (layer F.Cu) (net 1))
 (segment (start 134.62 144.78) (end 149.86 144.78) (width 0.5) (layer F.Cu) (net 1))
 (segment (start 126.746 123.19) (end 128.016 121.92) (width 0.5) (layer F.Cu) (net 1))
 (segment (start 126.746 128.27) (end 126.746 123.19) (width 0.5) (layer F.Cu) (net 1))
 (segment (start 124.333 130.683) (end 126.746 128.27) (width 0.5) (layer F.Cu) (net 1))
 (segment (start 124.333 140.462) (end 124.333 130.683) (width 0.5) (layer F.Cu) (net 1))
 (segment (start 128.651 144.78) (end 124.333 140.462) (width 0.5) (layer F.Cu) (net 1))
 (segment (start 134.62 144.78) (end 128.651 144.78) (width 0.5) (layer F.Cu) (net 1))
 (segment (start 141.66299 135.19701) (end 134.62 142.24) (width 0.25) (layer F.Cu) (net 12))
 (segment (start 141.66299 135.19701) (end 157.15699 135.19701) (width 0.25) (layer F.Cu) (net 12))
 (segment (start 161.544 130.81) (end 163.83 130.81) (width 0.25) (layer F.Cu) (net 12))
 (segment (start 157.15699 135.19701) (end 161.544 130.81) (width 0.25) (layer F.Cu) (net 12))
 (segment (start 163.83 128.27) (end 161.925 128.27) (width 0.25) (layer F.Cu) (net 11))
 (segment (start 161.925 128.27) (end 155.829 134.366) (width 0.25) (layer F.Cu) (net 11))
 (segment (start 139.954 134.366) (end 134.62 139.7) (width 0.25) (layer F.Cu) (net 11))
 (segment (start 155.829 134.366) (end 139.954 134.366) (width 0.25) (layer F.Cu) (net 11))
 (segment (start 162.7047 125.73) (end 155.0847 133.35) (width 0.25) (layer F.Cu) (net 16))
 (segment (start 163.83 125.73) (end 162.7047 125.73) (width 0.25) (layer F.Cu) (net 16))
 (segment (start 155.0847 133.35) (end 126.746 133.35) (width 0.25) (layer F.Cu) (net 16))
 (segment (start 163.83 123.19) (end 156.21 130.81) (width 0.25) (layer F.Cu) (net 17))
 (segment (start 156.21 130.81) (end 126.746 130.81) (width 0.25) (layer F.Cu) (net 17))
 (segment (start 153.67 118.11) (end 151.13 118.11) (width 0.25) (layer F.Cu) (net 15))
 (segment (start 161.29 118.11) (end 163.83 120.65) (width 0.25) (layer F.Cu) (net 15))
 (segment (start 153.67 118.11) (end 161.29 118.11) (width 0.25) (layer F.Cu) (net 15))
 (segment (start 162.654999 116.934999) (end 163.83 118.11) (width 0.25) (layer F.Cu) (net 14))
 (segment (start 138.335001 116.934999) (end 162.654999 116.934999) (width 0.25) (layer F.Cu) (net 14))
 (segment (start 135.89 119.38) (end 138.335001 116.934999) (width 0.25) (layer F.Cu) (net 14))
 (segment (start 138.335001 114.394999) (end 135.89 116.84) (width 0.25) (layer F.Cu) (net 13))
 (segment (start 162.654999 114.394999) (end 138.335001 114.394999) (width 0.25) (layer F.Cu) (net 13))
 (segment (start 163.83 115.57) (end 162.654999 114.394999) (width 0.25) (layer F.Cu) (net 13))
 (segment (start 154.0374 95.1553) (end 153.67 95.1553) (width 0.25) (layer B.Cu) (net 2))
 (segment (start 153.67 95.25) (end 151.13 95.25) (width 0.25) (layer F.Cu) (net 2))
 (segment (start 163.83 107.95) (end 160.655 107.95) (width 0.25) (layer F.Cu) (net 2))
 (segment (start 160.655 107.95) (end 158.242 105.537) (width 0.25) (layer F.Cu) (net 2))
 (segment (start 158.242 99.822) (end 153.67 95.25) (width 0.25) (layer F.Cu) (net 2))
 (segment (start 158.242 105.537) (end 158.242 99.822) (width 0.25) (layer F.Cu) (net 2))
 (segment (start 135.89 95.25) (end 133.35 95.25) (width 0.25) (layer F.Cu) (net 18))
 (segment (start 137.065001 94.074999) (end 135.89 95.25) (width 0.25) (layer F.Cu) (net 18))
 (segment (start 154.234001 94.074999) (end 137.065001 94.074999) (width 0.25) (layer F.Cu) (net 18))
 (segment (start 163.83 103.670998) (end 154.234001 94.074999) (width 0.25) (layer F.Cu) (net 18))
 (segment (start 163.83 105.41) (end 163.83 103.670998) (width 0.25) (layer F.Cu) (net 18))
 (segment (start 135.89 97.79) (end 148.6847 97.79) (width 0.25) (layer F.Cu) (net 3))
 (segment (start 133.35 97.79) (end 135.89 97.79) (width 0.25) (layer F.Cu) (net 3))
 (segment (start 148.6847 97.79) (end 153.67 97.79) (width 0.25) (layer F.Cu) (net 3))
 (segment (start 135.89 100.33) (end 133.35 100.33) (width 0.25) (layer F.Cu) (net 19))
 (segment (start 151.13 100.33) (end 153.67 100.33) (width 0.25) (layer F.Cu) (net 4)))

